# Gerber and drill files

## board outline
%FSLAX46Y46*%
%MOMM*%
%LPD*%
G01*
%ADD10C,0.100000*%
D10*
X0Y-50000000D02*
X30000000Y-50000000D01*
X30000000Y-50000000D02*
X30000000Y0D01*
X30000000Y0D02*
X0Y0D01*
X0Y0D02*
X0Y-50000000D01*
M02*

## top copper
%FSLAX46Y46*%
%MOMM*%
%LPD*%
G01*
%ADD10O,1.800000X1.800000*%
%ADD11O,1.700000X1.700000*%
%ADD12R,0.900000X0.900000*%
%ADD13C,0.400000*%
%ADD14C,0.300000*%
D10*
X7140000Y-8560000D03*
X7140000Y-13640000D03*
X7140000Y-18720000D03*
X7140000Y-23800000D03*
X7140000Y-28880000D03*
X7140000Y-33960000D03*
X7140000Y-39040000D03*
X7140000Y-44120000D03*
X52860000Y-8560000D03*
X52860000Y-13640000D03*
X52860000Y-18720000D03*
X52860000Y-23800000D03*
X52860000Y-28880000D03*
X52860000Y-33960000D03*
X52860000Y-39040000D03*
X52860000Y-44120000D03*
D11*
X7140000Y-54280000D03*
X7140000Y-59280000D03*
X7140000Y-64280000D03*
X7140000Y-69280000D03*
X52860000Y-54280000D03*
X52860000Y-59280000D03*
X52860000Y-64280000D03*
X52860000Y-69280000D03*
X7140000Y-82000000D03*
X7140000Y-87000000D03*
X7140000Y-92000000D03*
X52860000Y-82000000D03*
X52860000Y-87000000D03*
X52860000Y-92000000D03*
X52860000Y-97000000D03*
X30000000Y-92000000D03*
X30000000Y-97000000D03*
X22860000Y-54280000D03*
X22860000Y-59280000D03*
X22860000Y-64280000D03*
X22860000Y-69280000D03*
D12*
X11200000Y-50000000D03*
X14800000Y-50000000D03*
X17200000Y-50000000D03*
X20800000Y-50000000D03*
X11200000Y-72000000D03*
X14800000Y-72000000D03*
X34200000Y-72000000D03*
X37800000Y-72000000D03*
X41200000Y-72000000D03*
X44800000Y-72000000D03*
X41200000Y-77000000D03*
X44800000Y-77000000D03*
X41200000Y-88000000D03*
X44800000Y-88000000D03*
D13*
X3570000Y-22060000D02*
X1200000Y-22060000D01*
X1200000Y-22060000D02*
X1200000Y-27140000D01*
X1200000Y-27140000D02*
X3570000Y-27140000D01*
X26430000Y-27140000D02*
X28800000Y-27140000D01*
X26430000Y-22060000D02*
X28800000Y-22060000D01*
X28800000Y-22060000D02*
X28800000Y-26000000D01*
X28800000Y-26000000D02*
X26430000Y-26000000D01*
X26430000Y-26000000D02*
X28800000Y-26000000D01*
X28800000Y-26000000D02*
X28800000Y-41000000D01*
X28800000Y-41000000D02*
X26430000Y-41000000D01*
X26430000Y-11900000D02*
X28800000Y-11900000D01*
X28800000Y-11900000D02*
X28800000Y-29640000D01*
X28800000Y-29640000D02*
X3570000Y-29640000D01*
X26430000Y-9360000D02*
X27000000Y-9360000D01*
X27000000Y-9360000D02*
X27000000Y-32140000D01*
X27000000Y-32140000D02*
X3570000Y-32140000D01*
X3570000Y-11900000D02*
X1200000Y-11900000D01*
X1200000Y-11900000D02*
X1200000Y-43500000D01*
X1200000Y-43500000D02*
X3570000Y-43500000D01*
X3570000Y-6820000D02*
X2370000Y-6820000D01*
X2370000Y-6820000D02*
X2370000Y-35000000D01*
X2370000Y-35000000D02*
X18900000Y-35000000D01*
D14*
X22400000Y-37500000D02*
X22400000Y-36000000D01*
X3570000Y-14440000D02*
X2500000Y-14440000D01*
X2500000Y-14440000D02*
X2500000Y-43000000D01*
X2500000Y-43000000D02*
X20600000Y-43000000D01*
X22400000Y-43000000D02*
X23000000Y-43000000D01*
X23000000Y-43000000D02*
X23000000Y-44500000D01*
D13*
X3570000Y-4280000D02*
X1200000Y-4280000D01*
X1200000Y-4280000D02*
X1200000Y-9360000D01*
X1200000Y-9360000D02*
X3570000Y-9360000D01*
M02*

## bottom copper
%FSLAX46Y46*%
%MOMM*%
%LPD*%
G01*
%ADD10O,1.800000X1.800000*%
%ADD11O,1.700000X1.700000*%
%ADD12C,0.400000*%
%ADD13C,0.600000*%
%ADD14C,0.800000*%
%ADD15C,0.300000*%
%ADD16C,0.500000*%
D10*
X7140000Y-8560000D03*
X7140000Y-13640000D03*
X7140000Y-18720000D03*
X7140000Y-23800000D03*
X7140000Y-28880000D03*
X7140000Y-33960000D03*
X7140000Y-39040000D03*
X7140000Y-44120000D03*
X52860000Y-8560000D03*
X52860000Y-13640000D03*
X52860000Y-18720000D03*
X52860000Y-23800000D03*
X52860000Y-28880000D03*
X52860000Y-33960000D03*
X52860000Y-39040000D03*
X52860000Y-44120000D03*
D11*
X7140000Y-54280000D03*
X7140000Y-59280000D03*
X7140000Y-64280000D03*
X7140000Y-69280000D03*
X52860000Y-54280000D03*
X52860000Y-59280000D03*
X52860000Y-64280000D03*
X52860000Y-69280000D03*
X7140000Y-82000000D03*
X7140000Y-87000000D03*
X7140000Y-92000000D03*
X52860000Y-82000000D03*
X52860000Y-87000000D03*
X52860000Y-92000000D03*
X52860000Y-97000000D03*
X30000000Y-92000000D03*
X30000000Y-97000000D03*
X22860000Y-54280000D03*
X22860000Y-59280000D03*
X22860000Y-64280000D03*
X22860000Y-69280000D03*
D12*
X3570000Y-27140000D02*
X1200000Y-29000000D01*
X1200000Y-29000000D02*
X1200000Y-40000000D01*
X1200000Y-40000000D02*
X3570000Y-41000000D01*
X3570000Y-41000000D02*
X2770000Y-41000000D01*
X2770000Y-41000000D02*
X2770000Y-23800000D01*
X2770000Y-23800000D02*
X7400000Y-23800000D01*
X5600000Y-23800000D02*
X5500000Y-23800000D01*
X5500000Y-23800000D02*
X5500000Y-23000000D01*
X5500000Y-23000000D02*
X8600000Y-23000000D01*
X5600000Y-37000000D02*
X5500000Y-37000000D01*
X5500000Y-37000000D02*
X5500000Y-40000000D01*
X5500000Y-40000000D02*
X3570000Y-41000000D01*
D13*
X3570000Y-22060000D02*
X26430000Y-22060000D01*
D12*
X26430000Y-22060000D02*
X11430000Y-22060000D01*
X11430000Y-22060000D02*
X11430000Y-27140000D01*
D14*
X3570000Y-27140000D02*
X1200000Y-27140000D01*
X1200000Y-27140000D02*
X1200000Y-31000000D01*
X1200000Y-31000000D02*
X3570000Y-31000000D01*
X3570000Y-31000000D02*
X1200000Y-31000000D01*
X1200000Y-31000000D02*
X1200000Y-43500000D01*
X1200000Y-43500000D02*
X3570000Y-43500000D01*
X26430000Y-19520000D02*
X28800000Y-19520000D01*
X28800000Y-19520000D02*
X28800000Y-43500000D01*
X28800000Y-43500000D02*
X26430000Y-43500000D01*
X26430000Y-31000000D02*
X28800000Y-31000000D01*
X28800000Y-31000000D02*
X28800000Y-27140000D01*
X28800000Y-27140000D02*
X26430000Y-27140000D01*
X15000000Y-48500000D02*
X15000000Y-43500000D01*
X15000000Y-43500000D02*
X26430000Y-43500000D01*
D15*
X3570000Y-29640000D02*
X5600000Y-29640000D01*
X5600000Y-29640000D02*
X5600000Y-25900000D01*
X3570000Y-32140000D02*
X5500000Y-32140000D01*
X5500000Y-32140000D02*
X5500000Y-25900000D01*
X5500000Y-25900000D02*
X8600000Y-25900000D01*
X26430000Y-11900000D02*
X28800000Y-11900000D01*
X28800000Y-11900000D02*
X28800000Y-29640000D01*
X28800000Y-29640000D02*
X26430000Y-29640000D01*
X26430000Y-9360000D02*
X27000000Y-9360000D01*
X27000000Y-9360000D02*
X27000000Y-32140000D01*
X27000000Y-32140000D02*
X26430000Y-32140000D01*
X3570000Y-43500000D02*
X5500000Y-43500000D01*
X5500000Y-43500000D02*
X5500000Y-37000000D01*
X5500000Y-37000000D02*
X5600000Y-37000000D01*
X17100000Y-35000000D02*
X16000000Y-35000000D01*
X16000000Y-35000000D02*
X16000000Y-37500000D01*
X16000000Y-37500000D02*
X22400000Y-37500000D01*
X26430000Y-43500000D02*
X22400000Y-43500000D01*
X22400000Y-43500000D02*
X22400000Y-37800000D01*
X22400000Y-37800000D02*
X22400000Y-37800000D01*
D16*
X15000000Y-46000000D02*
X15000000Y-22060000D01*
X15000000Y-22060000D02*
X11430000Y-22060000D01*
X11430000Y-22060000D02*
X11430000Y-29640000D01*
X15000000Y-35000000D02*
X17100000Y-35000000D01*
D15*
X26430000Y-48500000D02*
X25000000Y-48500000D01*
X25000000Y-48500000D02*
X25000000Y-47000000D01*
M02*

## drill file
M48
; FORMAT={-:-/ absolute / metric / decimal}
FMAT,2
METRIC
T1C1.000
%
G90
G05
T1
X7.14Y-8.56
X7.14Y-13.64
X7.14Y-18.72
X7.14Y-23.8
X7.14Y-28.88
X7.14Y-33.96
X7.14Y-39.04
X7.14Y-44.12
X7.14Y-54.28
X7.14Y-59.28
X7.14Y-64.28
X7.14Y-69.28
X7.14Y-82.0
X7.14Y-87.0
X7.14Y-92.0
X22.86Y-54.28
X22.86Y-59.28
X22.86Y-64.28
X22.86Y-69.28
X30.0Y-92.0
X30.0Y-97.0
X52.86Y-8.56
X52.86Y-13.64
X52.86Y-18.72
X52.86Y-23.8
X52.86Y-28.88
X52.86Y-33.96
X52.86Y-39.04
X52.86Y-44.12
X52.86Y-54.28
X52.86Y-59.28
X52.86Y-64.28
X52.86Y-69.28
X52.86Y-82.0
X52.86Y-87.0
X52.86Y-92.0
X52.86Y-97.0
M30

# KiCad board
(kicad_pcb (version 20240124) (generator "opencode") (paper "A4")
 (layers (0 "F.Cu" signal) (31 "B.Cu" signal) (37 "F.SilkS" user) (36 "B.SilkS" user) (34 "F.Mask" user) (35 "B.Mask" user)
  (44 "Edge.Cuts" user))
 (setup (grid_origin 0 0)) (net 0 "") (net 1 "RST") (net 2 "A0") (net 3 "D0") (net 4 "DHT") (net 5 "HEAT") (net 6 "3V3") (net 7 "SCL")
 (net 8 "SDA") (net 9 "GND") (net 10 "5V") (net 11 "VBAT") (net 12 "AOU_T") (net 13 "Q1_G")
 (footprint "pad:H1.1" (layer "F.Cu") (at 3.57 4.28 0)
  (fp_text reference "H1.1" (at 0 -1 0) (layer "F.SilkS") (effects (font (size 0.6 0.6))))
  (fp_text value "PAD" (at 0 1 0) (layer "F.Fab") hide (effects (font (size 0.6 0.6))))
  (pad "1" thru_hole oval (at 3.57 4.28) (size 1.80 1.80) (drill 1.00) (layers *.Cu *.Mask) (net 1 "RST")))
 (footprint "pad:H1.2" (layer "F.Cu") (at 3.57 6.82 0)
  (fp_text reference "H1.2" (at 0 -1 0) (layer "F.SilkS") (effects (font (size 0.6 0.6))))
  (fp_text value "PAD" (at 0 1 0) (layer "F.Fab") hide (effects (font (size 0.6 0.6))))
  (pad "1" thru_hole oval (at 3.57 6.82) (size 1.80 1.80) (drill 1.00) (layers *.Cu *.Mask) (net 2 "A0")))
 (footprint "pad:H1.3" (layer "F.Cu") (at 3.57 9.36 0)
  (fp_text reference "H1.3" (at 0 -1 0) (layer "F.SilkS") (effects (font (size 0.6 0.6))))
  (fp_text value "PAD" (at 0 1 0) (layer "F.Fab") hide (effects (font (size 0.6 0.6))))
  (pad "1" thru_hole oval (at 3.57 9.36) (size 1.80 1.80) (drill 1.00) (layers *.Cu *.Mask) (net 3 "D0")))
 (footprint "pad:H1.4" (layer "F.Cu") (at 3.57 11.90 0)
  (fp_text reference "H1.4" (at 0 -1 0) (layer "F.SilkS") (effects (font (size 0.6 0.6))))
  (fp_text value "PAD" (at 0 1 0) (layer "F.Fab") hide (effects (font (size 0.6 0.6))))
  (pad "1" thru_hole oval (at 3.57 11.90) (size 1.80 1.80) (drill 1.00) (layers *.Cu *.Mask) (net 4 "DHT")))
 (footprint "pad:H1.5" (layer "F.Cu") (at 3.57 14.44 0)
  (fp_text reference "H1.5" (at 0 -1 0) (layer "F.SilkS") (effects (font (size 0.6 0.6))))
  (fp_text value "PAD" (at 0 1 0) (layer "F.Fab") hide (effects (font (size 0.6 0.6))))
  (pad "1" thru_hole oval (at 3.57 14.44) (size 1.80 1.80) (drill 1.00) (layers *.Cu *.Mask) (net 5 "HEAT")))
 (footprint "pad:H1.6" (layer "F.Cu") (at 3.57 16.98 0)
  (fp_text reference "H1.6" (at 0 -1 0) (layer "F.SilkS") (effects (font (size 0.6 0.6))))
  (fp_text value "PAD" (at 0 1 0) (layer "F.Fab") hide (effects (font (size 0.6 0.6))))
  (pad "1" thru_hole oval (at 3.57 16.98) (size 1.80 1.80) (drill 1.00) (layers *.Cu *.Mask) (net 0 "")))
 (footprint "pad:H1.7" (layer "F.Cu") (at 3.57 19.52 0)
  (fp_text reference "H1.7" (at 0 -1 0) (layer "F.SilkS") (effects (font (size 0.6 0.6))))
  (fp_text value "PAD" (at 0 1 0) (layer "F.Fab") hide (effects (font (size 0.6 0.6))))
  (pad "1" thru_hole oval (at 3.57 19.52) (size 1.80 1.80) (drill 1.00) (layers *.Cu *.Mask) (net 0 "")))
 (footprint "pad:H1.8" (layer "F.Cu") (at 3.57 22.06 0)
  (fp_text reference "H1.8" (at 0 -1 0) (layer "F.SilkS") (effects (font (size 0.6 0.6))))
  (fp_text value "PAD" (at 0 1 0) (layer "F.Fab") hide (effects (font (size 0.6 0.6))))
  (pad "1" thru_hole oval (at 3.57 22.06) (size 1.80 1.80) (drill 1.00) (layers *.Cu *.Mask) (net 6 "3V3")))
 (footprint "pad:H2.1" (layer "F.Cu") (at 26.43 4.28 0)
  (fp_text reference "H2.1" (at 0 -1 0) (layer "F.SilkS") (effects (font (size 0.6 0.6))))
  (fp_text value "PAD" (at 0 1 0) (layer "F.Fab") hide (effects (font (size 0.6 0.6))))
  (pad "1" thru_hole oval (at 26.43 4.28) (size 1.80 1.80) (drill 1.00) (layers *.Cu *.Mask) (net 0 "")))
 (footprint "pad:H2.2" (layer "F.Cu") (at 26.43 6.82 0)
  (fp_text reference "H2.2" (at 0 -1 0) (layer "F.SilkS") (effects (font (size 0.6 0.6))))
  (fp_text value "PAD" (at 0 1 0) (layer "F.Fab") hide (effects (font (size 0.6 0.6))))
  (pad "1" thru_hole oval (at 26.43 6.82) (size 1.80 1.80) (drill 1.00) (layers *.Cu *.Mask) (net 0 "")))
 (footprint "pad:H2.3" (layer "F.Cu") (at 26.43 9.36 0)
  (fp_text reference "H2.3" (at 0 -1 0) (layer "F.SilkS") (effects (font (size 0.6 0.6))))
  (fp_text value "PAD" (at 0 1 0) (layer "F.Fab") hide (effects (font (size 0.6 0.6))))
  (pad "1" thru_hole oval (at 26.43 9.36) (size 1.80 1.80) (drill 1.00) (layers *.Cu *.Mask) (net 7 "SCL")))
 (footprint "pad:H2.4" (layer "F.Cu") (at 26.43 11.90 0)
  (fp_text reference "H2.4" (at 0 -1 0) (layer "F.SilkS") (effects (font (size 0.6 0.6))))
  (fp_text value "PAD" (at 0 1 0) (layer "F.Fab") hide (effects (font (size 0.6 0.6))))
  (pad "1" thru_hole oval (at 26.43 11.90) (size 1.80 1.80) (drill 1.00) (layers *.Cu *.Mask) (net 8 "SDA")))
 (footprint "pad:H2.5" (layer "F.Cu") (at 26.43 14.44 0)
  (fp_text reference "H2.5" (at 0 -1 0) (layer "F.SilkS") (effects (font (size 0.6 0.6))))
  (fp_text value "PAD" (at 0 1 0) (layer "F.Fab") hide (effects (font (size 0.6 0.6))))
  (pad "1" thru_hole oval (at 26.43 14.44) (size 1.80 1.80) (drill 1.00) (layers *.Cu *.Mask) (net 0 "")))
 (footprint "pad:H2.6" (layer "F.Cu") (at 26.43 16.98 0)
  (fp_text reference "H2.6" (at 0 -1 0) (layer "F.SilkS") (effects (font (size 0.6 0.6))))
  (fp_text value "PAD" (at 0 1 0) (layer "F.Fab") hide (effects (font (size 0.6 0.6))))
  (pad "1" thru_hole oval (at 26.43 16.98) (size 1.80 1.80) (drill 1.00) (layers *.Cu *.Mask) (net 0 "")))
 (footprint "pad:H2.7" (layer "F.Cu") (at 26.43 19.52 0)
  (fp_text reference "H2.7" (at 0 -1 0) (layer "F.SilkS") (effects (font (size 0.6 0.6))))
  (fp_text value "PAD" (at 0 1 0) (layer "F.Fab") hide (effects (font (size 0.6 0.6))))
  (pad "1" thru_hole oval (at 26.43 19.52) (size 1.80 1.80) (drill 1.00) (layers *.Cu *.Mask) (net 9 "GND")))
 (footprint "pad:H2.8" (layer "F.Cu") (at 26.43 22.06 0)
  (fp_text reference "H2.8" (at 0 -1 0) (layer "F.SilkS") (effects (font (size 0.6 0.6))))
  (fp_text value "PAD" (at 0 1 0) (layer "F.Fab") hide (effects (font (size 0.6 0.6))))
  (pad "1" thru_hole oval (at 26.43 22.06) (size 1.80 1.80) (drill 1.00) (layers *.Cu *.Mask) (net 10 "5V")))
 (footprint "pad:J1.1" (layer "F.Cu") (at 3.57 27.14 0)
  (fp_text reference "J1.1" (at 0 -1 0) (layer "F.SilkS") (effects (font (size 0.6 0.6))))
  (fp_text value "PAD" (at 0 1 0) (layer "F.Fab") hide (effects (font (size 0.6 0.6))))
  (pad "1" thru_hole oval (at 3.57 27.14) (size 1.70 1.70) (drill 1.00) (layers *.Cu *.Mask) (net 9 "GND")))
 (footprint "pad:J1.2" (layer "F.Cu") (at 3.57 29.64 0)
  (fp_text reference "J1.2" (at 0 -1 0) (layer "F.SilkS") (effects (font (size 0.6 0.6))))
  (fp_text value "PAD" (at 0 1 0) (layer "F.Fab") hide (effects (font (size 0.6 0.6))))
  (pad "1" thru_hole oval (at 3.57 29.64) (size 1.70 1.70) (drill 1.00) (layers *.Cu *.Mask) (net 6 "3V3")))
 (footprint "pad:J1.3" (layer "F.Cu") (at 3.57 32.14 0)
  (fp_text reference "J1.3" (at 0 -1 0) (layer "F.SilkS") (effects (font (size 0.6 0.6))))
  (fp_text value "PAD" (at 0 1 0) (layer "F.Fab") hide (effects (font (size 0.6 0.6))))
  (pad "1" thru_hole oval (at 3.57 32.14) (size 1.70 1.70) (drill 1.00) (layers *.Cu *.Mask) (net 8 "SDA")))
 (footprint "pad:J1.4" (layer "F.Cu") (at 3.57 34.64 0)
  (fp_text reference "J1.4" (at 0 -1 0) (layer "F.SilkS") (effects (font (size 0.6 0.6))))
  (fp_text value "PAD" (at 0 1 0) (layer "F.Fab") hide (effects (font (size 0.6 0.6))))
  (pad "1" thru_hole oval (at 3.57 34.64) (size 1.70 1.70) (drill 1.00) (layers *.Cu *.Mask) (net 7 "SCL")))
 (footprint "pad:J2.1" (layer "F.Cu") (at 26.43 27.14 0)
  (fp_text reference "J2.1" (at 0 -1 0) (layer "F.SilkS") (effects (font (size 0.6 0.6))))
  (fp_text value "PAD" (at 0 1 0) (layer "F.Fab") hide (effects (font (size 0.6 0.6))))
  (pad "1" thru_hole oval (at 26.43 27.14) (size 1.70 1.70) (drill 1.00) (layers *.Cu *.Mask) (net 9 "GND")))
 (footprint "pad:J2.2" (layer "F.Cu") (at 26.43 29.64 0)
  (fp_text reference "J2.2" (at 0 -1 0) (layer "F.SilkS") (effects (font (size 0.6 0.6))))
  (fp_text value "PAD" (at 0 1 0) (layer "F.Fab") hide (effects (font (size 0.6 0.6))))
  (pad "1" thru_hole oval (at 26.43 29.64) (size 1.70 1.70) (drill 1.00) (layers *.Cu *.Mask) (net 6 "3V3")))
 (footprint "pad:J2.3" (layer "F.Cu") (at 26.43 32.14 0)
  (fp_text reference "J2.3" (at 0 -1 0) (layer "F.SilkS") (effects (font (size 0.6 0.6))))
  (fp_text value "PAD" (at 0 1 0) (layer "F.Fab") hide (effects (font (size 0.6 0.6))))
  (pad "1" thru_hole oval (at 26.43 32.14) (size 1.70 1.70) (drill 1.00) (layers *.Cu *.Mask) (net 8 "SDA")))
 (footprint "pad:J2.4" (layer "F.Cu") (at 26.43 34.64 0)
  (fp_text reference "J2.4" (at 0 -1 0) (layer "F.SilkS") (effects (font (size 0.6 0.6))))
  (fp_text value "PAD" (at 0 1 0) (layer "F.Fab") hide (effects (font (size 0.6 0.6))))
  (pad "1" thru_hole oval (at 26.43 34.64) (size 1.70 1.70) (drill 1.00) (layers *.Cu *.Mask) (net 7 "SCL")))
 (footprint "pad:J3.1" (layer "F.Cu") (at 3.57 41.00 0)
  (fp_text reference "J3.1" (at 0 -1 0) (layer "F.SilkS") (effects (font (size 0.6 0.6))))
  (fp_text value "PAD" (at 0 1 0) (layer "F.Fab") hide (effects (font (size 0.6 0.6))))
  (pad "1" thru_hole oval (at 3.57 41.00) (size 1.70 1.70) (drill 1.00) (layers *.Cu *.Mask) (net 6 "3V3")))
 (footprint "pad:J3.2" (layer "F.Cu") (at 3.57 43.50 0)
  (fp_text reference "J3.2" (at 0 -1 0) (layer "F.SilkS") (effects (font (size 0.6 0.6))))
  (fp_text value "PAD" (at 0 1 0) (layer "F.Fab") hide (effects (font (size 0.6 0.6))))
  (pad "1" thru_hole oval (at 3.57 43.50) (size 1.70 1.70) (drill 1.00) (layers *.Cu *.Mask) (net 4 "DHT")))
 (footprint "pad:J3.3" (layer "F.Cu") (at 3.57 46.00 0)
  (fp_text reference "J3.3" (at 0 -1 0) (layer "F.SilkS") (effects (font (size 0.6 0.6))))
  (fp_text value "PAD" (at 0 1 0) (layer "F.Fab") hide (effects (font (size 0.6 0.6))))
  (pad "1" thru_hole oval (at 3.57 46.00) (size 1.70 1.70) (drill 1.00) (layers *.Cu *.Mask) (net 9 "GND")))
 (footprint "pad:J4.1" (layer "F.Cu") (at 26.43 41.00 0)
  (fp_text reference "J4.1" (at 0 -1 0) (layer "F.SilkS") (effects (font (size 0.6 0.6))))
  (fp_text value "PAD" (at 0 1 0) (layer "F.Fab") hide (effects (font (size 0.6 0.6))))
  (pad "1" thru_hole oval (at 26.43 41.00) (size 1.70 1.70) (drill 1.00) (layers *.Cu *.Mask) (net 10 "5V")))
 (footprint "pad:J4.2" (layer "F.Cu") (at 26.43 43.50 0)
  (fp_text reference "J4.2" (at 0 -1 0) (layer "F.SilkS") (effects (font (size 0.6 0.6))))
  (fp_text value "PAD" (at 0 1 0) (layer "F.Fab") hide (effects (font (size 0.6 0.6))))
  (pad "1" thru_hole oval (at 26.43 43.50) (size 1.70 1.70) (drill 1.00) (layers *.Cu *.Mask) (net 9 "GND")))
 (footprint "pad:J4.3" (layer "F.Cu") (at 26.43 46.00 0)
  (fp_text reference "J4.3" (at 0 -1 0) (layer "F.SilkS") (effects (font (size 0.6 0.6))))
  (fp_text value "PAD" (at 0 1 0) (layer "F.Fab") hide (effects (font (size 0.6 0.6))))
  (pad "1" thru_hole oval (at 26.43 46.00) (size 1.70 1.70) (drill 1.00) (layers *.Cu *.Mask) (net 2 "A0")))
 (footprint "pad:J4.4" (layer "F.Cu") (at 26.43 48.50 0)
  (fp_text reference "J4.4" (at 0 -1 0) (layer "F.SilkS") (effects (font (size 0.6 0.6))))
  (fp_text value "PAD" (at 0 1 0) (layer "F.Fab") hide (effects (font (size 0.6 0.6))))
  (pad "1" thru_hole oval (at 26.43 48.50) (size 1.70 1.70) (drill 1.00) (layers *.Cu *.Mask) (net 5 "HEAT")))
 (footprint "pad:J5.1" (layer "F.Cu") (at 15.00 46.00 0)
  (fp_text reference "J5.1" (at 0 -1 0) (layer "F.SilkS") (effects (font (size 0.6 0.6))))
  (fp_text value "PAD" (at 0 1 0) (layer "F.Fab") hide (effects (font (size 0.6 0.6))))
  (pad "1" thru_hole oval (at 15.00 46.00) (size 1.70 1.70) (drill 1.00) (layers *.Cu *.Mask) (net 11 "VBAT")))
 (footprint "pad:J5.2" (layer "F.Cu") (at 15.00 48.50 0)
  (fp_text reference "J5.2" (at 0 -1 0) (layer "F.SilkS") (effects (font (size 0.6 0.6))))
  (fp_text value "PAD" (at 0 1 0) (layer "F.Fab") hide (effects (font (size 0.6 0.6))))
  (pad "1" thru_hole oval (at 15.00 48.50) (size 1.70 1.70) (drill 1.00) (layers *.Cu *.Mask) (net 9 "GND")))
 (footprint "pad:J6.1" (layer "F.Cu") (at 11.43 27.14 0)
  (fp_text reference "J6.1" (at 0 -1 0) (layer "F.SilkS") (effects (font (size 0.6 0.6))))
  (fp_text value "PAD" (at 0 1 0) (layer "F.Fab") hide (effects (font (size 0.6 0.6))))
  (pad "1" thru_hole oval (at 11.43 27.14) (size 1.70 1.70) (drill 1.00) (layers *.Cu *.Mask) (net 10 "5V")))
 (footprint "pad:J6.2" (layer "F.Cu") (at 11.43 29.64 0)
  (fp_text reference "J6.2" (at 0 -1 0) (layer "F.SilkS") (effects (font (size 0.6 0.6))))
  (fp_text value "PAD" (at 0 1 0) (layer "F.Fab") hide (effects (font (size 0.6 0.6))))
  (pad "1" thru_hole oval (at 11.43 29.64) (size 1.70 1.70) (drill 1.00) (layers *.Cu *.Mask) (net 9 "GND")))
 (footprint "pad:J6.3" (layer "F.Cu") (at 11.43 32.14 0)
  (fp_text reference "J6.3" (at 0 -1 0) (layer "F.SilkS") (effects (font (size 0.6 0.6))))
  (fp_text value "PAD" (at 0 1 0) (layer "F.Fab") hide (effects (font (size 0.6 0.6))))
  (pad "1" thru_hole oval (at 11.43 32.14) (size 1.70 1.70) (drill 1.00) (layers *.Cu *.Mask) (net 11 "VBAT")))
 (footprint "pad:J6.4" (layer "F.Cu") (at 11.43 34.64 0)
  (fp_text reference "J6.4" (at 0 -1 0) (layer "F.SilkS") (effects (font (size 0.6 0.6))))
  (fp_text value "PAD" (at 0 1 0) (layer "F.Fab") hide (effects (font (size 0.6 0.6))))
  (pad "1" thru_hole oval (at 11.43 34.64) (size 1.70 1.70) (drill 1.00) (layers *.Cu *.Mask) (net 9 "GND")))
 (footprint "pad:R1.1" (layer "F.Cu") (at 5.60 25.00 0)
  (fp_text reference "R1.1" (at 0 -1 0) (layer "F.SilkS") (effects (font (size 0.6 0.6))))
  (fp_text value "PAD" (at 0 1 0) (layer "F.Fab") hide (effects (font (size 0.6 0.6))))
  (pad "1" smd rect (at 5.60 25.00) (size 0.90 0.90) (layers F.Cu F.Paste F.Mask) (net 6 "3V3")))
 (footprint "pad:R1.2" (layer "F.Cu") (at 7.40 25.00 0)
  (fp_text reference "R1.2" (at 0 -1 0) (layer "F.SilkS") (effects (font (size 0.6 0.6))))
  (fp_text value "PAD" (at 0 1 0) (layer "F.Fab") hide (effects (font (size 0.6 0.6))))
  (pad "1" smd rect (at 7.40 25.00) (size 0.90 0.90) (layers F.Cu F.Paste F.Mask) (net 8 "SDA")))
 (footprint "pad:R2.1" (layer "F.Cu") (at 8.60 25.00 0)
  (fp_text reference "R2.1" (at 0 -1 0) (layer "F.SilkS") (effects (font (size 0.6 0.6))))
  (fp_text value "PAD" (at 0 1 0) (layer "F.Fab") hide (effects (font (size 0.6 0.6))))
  (pad "1" smd rect (at 8.60 25.00) (size 0.90 0.90) (layers F.Cu F.Paste F.Mask) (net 6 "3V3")))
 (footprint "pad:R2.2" (layer "F.Cu") (at 10.40 25.00 0)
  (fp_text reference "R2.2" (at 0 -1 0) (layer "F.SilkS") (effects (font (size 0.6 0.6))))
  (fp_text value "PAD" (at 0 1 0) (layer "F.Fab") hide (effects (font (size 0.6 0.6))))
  (pad "1" smd rect (at 10.40 25.00) (size 0.90 0.90) (layers F.Cu F.Paste F.Mask) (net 7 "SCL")))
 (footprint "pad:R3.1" (layer "F.Cu") (at 5.60 36.00 0)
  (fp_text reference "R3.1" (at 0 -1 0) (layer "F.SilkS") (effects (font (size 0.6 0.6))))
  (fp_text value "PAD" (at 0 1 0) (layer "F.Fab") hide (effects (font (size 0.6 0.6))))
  (pad "1" smd rect (at 5.60 36.00) (size 0.90 0.90) (layers F.Cu F.Paste F.Mask) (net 6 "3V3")))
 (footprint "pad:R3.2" (layer "F.Cu") (at 7.40 36.00 0)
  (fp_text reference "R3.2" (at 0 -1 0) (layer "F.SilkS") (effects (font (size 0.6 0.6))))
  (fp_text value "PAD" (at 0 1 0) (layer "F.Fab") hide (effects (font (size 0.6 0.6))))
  (pad "1" smd rect (at 7.40 36.00) (size 0.90 0.90) (layers F.Cu F.Paste F.Mask) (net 4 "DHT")))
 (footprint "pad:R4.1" (layer "F.Cu") (at 17.10 36.00 0)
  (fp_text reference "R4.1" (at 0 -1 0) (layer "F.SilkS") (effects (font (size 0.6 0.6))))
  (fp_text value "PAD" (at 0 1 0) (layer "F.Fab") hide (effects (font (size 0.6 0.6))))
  (pad "1" smd rect (at 17.10 36.00) (size 0.90 0.90) (layers F.Cu F.Paste F.Mask) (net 11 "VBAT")))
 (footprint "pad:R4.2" (layer "F.Cu") (at 18.90 36.00 0)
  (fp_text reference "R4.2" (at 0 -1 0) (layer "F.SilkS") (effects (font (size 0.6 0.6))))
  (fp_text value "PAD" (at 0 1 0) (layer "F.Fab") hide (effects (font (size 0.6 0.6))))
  (pad "1" smd rect (at 18.90 36.00) (size 0.90 0.90) (layers F.Cu F.Paste F.Mask) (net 2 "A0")))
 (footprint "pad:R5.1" (layer "F.Cu") (at 20.60 36.00 0)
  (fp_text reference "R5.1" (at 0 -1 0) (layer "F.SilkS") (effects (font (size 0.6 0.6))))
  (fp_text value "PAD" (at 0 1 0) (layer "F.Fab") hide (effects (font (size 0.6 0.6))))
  (pad "1" smd rect (at 20.60 36.00) (size 0.90 0.90) (layers F.Cu F.Paste F.Mask) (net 2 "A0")))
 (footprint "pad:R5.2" (layer "F.Cu") (at 22.40 36.00 0)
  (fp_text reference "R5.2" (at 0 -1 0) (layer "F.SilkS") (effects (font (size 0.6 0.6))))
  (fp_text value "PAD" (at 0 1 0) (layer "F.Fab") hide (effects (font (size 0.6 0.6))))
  (pad "1" smd rect (at 22.40 36.00) (size 0.90 0.90) (layers F.Cu F.Paste F.Mask) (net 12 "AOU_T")))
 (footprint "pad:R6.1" (layer "F.Cu") (at 20.60 38.50 0)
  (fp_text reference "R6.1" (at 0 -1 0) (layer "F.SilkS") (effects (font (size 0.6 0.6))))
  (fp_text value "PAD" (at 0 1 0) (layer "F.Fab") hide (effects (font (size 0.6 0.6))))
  (pad "1" smd rect (at 20.60 38.50) (size 0.90 0.90) (layers F.Cu F.Paste F.Mask) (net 12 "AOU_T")))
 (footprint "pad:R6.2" (layer "F.Cu") (at 22.40 38.50 0)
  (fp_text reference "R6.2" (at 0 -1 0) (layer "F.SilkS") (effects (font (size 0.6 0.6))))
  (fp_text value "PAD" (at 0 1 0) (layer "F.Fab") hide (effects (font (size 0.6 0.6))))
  (pad "1" smd rect (at 22.40 38.50) (size 0.90 0.90) (layers F.Cu F.Paste F.Mask) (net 9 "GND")))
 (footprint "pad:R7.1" (layer "F.Cu") (at 20.60 44.00 0)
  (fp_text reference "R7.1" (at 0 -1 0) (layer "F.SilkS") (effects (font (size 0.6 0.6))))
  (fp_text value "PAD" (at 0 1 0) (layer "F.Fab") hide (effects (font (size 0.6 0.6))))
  (pad "1" smd rect (at 20.60 44.00) (size 0.90 0.90) (layers F.Cu F.Paste F.Mask) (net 5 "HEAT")))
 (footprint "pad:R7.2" (layer "F.Cu") (at 22.40 44.00 0)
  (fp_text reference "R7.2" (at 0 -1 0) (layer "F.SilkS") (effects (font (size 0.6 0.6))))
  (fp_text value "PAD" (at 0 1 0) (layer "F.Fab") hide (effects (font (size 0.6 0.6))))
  (pad "1" smd rect (at 22.40 44.00) (size 0.90 0.90) (layers F.Cu F.Paste F.Mask) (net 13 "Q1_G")))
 (segment (start 3.57 22.06) (end 1.20 22.06) (width 0.40) (layer "F.Cu") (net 6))
 (segment (start 1.20 22.06) (end 1.20 27.14) (width 0.40) (layer "F.Cu") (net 6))
 (segment (start 1.20 27.14) (end 3.57 27.14) (width 0.40) (layer "F.Cu") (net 6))
 (segment (start 3.57 27.14) (end 1.20 29.00) (width 0.40) (layer "B.Cu") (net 6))
 (segment (start 1.20 29.00) (end 1.20 40.00) (width 0.40) (layer "B.Cu") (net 6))
 (segment (start 1.20 40.00) (end 3.57 41.00) (width 0.40) (layer "B.Cu") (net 6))
 (segment (start 3.57 41.00) (end 2.77 41.00) (width 0.40) (layer "B.Cu") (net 6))
 (segment (start 2.77 41.00) (end 2.77 23.80) (width 0.40) (layer "B.Cu") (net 6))
 (segment (start 2.77 23.80) (end 7.40 23.80) (width 0.40) (layer "B.Cu") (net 6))
 (segment (start 5.60 23.80) (end 5.50 23.80) (width 0.40) (layer "B.Cu") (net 6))
 (segment (start 5.50 23.80) (end 5.50 23.00) (width 0.40) (layer "B.Cu") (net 6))
 (segment (start 5.50 23.00) (end 8.60 23.00) (width 0.40) (layer "B.Cu") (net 6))
 (segment (start 5.60 37.00) (end 5.50 37.00) (width 0.40) (layer "B.Cu") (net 6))
 (segment (start 5.50 37.00) (end 5.50 40.00) (width 0.40) (layer "B.Cu") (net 6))
 (segment (start 5.50 40.00) (end 3.57 41.00) (width 0.40) (layer "B.Cu") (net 6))
 (segment (start 26.43 27.14) (end 28.80 27.14) (width 0.40) (layer "F.Cu") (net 6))
 (segment (start 3.57 22.06) (end 26.43 22.06) (width 0.60) (layer "B.Cu") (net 6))
 (segment (start 26.43 22.06) (end 28.80 22.06) (width 0.40) (layer "F.Cu") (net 10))
 (segment (start 28.80 22.06) (end 28.80 26.00) (width 0.40) (layer "F.Cu") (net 10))
 (segment (start 28.80 26.00) (end 26.43 26.00) (width 0.40) (layer "F.Cu") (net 10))
 (segment (start 26.43 26.00) (end 28.80 26.00) (width 0.40) (layer "F.Cu") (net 10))
 (segment (start 28.80 26.00) (end 28.80 41.00) (width 0.40) (layer "F.Cu") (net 10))
 (segment (start 28.80 41.00) (end 26.43 41.00) (width 0.40) (layer "F.Cu") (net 10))
 (segment (start 26.43 22.06) (end 11.43 22.06) (width 0.40) (layer "B.Cu") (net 10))
 (segment (start 11.43 22.06) (end 11.43 27.14) (width 0.40) (layer "B.Cu") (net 10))
 (segment (start 3.57 27.14) (end 1.20 27.14) (width 0.80) (layer "B.Cu") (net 9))
 (segment (start 1.20 27.14) (end 1.20 31.00) (width 0.80) (layer "B.Cu") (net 9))
 (segment (start 1.20 31.00) (end 3.57 31.00) (width 0.80) (layer "B.Cu") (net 9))
 (segment (start 3.57 31.00) (end 1.20 31.00) (width 0.80) (layer "B.Cu") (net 9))
 (segment (start 1.20 31.00) (end 1.20 43.50) (width 0.80) (layer "B.Cu") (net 9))
 (segment (start 1.20 43.50) (end 3.57 43.50) (width 0.80) (layer "B.Cu") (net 9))
 (segment (start 26.43 19.52) (end 28.80 19.52) (width 0.80) (layer "B.Cu") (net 9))
 (segment (start 28.80 19.52) (end 28.80 43.50) (width 0.80) (layer "B.Cu") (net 9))
 (segment (start 28.80 43.50) (end 26.43 43.50) (width 0.80) (layer "B.Cu") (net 9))
 (segment (start 26.43 31.00) (end 28.80 31.00) (width 0.80) (layer "B.Cu") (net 9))
 (segment (start 28.80 31.00) (end 28.80 27.14) (width 0.80) (layer "B.Cu") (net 9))
 (segment (start 28.80 27.14) (end 26.43 27.14) (width 0.80) (layer "B.Cu") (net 9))
 (segment (start 15.00 48.50) (end 15.00 43.50) (width 0.80) (layer "B.Cu") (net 9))
 (segment (start 15.00 43.50) (end 26.43 43.50) (width 0.80) (layer "B.Cu") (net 9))
 (segment (start 26.43 11.90) (end 28.80 11.90) (width 0.40) (layer "F.Cu") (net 8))
 (segment (start 28.80 11.90) (end 28.80 29.64) (width 0.40) (layer "F.Cu") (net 8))
 (segment (start 28.80 29.64) (end 3.57 29.64) (width 0.40) (layer "F.Cu") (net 8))
 (segment (start 26.43 9.36) (end 27.00 9.36) (width 0.40) (layer "F.Cu") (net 7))
 (segment (start 27.00 9.36) (end 27.00 32.14) (width 0.40) (layer "F.Cu") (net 7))
 (segment (start 27.00 32.14) (end 3.57 32.14) (width 0.40) (layer "F.Cu") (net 7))
 (segment (start 3.57 29.64) (end 5.60 29.64) (width 0.30) (layer "B.Cu") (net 8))
 (segment (start 5.60 29.64) (end 5.60 25.90) (width 0.30) (layer "B.Cu") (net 8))
 (segment (start 3.57 32.14) (end 5.50 32.14) (width 0.30) (layer "B.Cu") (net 7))
 (segment (start 5.50 32.14) (end 5.50 25.90) (width 0.30) (layer "B.Cu") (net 7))
 (segment (start 5.50 25.90) (end 8.60 25.90) (width 0.30) (layer "B.Cu") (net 7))
 (segment (start 26.43 11.90) (end 28.80 11.90) (width 0.30) (layer "B.Cu") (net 8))
 (segment (start 28.80 11.90) (end 28.80 29.64) (width 0.30) (layer "B.Cu") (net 8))
 (segment (start 28.80 29.64) (end 26.43 29.64) (width 0.30) (layer "B.Cu") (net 8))
 (segment (start 26.43 9.36) (end 27.00 9.36) (width 0.30) (layer "B.Cu") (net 7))
 (segment (start 27.00 9.36) (end 27.00 32.14) (width 0.30) (layer "B.Cu") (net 7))
 (segment (start 27.00 32.14) (end 26.43 32.14) (width 0.30) (layer "B.Cu") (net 7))
 (segment (start 3.57 11.90) (end 1.20 11.90) (width 0.40) (layer "F.Cu") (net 4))
 (segment (start 1.20 11.90) (end 1.20 43.50) (width 0.40) (layer "F.Cu") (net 4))
 (segment (start 1.20 43.50) (end 3.57 43.50) (width 0.40) (layer "F.Cu") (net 4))
 (segment (start 3.57 43.50) (end 5.50 43.50) (width 0.30) (layer "B.Cu") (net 4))
 (segment (start 5.50 43.50) (end 5.50 37.00) (width 0.30) (layer "B.Cu") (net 4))
 (segment (start 5.50 37.00) (end 5.60 37.00) (width 0.30) (layer "B.Cu") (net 4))
 (segment (start 3.57 6.82) (end 2.37 6.82) (width 0.40) (layer "F.Cu") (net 2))
 (segment (start 2.37 6.82) (end 2.37 35.00) (width 0.40) (layer "F.Cu") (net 2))
 (segment (start 2.37 35.00) (end 18.90 35.00) (width 0.40) (layer "F.Cu") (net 2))
 (segment (start 17.10 35.00) (end 16.00 35.00) (width 0.30) (layer "B.Cu") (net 2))
 (segment (start 16.00 35.00) (end 16.00 37.50) (width 0.30) (layer "B.Cu") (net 2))
 (segment (start 16.00 37.50) (end 22.40 37.50) (width 0.30) (layer "B.Cu") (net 2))
 (segment (start 22.40 37.50) (end 22.40 36.00) (width 0.30) (layer "F.Cu") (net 2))
 (segment (start 26.43 43.50) (end 22.40 43.50) (width 0.30) (layer "B.Cu") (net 2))
 (segment (start 22.40 43.50) (end 22.40 37.80) (width 0.30) (layer "B.Cu") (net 2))
 (segment (start 22.40 37.80) (end 22.40 37.80) (width 0.30) (layer "B.Cu") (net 2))
 (segment (start 15.00 46.00) (end 15.00 22.06) (width 0.50) (layer "B.Cu") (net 11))
 (segment (start 15.00 22.06) (end 11.43 22.06) (width 0.50) (layer "B.Cu") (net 11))
 (segment (start 11.43 22.06) (end 11.43 29.64) (width 0.50) (layer "B.Cu") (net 11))
 (segment (start 15.00 35.00) (end 17.10 35.00) (width 0.50) (layer "B.Cu") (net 11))
 (segment (start 3.57 14.44) (end 2.50 14.44) (width 0.30) (layer "F.Cu") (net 5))
 (segment (start 2.50 14.44) (end 2.50 43.00) (width 0.30) (layer "F.Cu") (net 5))
 (segment (start 2.50 43.00) (end 20.60 43.00) (width 0.30) (layer "F.Cu") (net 5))
 (segment (start 22.40 43.00) (end 23.00 43.00) (width 0.30) (layer "F.Cu") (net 5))
 (segment (start 23.00 43.00) (end 23.00 44.50) (width 0.30) (layer "F.Cu") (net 5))
 (segment (start 26.43 48.50) (end 25.00 48.50) (width 0.30) (layer "B.Cu") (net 5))
 (segment (start 25.00 48.50) (end 25.00 47.00) (width 0.30) (layer "B.Cu") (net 5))
 (segment (start 3.57 4.28) (end 1.20 4.28) (width 0.40) (layer "F.Cu") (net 1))
 (segment (start 1.20 4.28) (end 1.20 9.36) (width 0.40) (layer "F.Cu") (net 1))
 (segment (start 1.20 9.36) (end 3.57 9.36) (width 0.40) (layer "F.Cu") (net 1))
 (gr_line (start 0.00 50.00) (end 30.00 50.00) (layer "Edge.Cuts") (width 0.1))
 (gr_line (start 30.00 50.00) (end 30.00 0.00) (layer "Edge.Cuts") (width 0.1))
 (gr_line (start 30.00 0.00) (end 0.00 0.00) (layer "Edge.Cuts") (width 0.1))
 (gr_line (start 0.00 0.00) (end 0.00 50.00) (layer "Edge.Cuts") (width 0.1)))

